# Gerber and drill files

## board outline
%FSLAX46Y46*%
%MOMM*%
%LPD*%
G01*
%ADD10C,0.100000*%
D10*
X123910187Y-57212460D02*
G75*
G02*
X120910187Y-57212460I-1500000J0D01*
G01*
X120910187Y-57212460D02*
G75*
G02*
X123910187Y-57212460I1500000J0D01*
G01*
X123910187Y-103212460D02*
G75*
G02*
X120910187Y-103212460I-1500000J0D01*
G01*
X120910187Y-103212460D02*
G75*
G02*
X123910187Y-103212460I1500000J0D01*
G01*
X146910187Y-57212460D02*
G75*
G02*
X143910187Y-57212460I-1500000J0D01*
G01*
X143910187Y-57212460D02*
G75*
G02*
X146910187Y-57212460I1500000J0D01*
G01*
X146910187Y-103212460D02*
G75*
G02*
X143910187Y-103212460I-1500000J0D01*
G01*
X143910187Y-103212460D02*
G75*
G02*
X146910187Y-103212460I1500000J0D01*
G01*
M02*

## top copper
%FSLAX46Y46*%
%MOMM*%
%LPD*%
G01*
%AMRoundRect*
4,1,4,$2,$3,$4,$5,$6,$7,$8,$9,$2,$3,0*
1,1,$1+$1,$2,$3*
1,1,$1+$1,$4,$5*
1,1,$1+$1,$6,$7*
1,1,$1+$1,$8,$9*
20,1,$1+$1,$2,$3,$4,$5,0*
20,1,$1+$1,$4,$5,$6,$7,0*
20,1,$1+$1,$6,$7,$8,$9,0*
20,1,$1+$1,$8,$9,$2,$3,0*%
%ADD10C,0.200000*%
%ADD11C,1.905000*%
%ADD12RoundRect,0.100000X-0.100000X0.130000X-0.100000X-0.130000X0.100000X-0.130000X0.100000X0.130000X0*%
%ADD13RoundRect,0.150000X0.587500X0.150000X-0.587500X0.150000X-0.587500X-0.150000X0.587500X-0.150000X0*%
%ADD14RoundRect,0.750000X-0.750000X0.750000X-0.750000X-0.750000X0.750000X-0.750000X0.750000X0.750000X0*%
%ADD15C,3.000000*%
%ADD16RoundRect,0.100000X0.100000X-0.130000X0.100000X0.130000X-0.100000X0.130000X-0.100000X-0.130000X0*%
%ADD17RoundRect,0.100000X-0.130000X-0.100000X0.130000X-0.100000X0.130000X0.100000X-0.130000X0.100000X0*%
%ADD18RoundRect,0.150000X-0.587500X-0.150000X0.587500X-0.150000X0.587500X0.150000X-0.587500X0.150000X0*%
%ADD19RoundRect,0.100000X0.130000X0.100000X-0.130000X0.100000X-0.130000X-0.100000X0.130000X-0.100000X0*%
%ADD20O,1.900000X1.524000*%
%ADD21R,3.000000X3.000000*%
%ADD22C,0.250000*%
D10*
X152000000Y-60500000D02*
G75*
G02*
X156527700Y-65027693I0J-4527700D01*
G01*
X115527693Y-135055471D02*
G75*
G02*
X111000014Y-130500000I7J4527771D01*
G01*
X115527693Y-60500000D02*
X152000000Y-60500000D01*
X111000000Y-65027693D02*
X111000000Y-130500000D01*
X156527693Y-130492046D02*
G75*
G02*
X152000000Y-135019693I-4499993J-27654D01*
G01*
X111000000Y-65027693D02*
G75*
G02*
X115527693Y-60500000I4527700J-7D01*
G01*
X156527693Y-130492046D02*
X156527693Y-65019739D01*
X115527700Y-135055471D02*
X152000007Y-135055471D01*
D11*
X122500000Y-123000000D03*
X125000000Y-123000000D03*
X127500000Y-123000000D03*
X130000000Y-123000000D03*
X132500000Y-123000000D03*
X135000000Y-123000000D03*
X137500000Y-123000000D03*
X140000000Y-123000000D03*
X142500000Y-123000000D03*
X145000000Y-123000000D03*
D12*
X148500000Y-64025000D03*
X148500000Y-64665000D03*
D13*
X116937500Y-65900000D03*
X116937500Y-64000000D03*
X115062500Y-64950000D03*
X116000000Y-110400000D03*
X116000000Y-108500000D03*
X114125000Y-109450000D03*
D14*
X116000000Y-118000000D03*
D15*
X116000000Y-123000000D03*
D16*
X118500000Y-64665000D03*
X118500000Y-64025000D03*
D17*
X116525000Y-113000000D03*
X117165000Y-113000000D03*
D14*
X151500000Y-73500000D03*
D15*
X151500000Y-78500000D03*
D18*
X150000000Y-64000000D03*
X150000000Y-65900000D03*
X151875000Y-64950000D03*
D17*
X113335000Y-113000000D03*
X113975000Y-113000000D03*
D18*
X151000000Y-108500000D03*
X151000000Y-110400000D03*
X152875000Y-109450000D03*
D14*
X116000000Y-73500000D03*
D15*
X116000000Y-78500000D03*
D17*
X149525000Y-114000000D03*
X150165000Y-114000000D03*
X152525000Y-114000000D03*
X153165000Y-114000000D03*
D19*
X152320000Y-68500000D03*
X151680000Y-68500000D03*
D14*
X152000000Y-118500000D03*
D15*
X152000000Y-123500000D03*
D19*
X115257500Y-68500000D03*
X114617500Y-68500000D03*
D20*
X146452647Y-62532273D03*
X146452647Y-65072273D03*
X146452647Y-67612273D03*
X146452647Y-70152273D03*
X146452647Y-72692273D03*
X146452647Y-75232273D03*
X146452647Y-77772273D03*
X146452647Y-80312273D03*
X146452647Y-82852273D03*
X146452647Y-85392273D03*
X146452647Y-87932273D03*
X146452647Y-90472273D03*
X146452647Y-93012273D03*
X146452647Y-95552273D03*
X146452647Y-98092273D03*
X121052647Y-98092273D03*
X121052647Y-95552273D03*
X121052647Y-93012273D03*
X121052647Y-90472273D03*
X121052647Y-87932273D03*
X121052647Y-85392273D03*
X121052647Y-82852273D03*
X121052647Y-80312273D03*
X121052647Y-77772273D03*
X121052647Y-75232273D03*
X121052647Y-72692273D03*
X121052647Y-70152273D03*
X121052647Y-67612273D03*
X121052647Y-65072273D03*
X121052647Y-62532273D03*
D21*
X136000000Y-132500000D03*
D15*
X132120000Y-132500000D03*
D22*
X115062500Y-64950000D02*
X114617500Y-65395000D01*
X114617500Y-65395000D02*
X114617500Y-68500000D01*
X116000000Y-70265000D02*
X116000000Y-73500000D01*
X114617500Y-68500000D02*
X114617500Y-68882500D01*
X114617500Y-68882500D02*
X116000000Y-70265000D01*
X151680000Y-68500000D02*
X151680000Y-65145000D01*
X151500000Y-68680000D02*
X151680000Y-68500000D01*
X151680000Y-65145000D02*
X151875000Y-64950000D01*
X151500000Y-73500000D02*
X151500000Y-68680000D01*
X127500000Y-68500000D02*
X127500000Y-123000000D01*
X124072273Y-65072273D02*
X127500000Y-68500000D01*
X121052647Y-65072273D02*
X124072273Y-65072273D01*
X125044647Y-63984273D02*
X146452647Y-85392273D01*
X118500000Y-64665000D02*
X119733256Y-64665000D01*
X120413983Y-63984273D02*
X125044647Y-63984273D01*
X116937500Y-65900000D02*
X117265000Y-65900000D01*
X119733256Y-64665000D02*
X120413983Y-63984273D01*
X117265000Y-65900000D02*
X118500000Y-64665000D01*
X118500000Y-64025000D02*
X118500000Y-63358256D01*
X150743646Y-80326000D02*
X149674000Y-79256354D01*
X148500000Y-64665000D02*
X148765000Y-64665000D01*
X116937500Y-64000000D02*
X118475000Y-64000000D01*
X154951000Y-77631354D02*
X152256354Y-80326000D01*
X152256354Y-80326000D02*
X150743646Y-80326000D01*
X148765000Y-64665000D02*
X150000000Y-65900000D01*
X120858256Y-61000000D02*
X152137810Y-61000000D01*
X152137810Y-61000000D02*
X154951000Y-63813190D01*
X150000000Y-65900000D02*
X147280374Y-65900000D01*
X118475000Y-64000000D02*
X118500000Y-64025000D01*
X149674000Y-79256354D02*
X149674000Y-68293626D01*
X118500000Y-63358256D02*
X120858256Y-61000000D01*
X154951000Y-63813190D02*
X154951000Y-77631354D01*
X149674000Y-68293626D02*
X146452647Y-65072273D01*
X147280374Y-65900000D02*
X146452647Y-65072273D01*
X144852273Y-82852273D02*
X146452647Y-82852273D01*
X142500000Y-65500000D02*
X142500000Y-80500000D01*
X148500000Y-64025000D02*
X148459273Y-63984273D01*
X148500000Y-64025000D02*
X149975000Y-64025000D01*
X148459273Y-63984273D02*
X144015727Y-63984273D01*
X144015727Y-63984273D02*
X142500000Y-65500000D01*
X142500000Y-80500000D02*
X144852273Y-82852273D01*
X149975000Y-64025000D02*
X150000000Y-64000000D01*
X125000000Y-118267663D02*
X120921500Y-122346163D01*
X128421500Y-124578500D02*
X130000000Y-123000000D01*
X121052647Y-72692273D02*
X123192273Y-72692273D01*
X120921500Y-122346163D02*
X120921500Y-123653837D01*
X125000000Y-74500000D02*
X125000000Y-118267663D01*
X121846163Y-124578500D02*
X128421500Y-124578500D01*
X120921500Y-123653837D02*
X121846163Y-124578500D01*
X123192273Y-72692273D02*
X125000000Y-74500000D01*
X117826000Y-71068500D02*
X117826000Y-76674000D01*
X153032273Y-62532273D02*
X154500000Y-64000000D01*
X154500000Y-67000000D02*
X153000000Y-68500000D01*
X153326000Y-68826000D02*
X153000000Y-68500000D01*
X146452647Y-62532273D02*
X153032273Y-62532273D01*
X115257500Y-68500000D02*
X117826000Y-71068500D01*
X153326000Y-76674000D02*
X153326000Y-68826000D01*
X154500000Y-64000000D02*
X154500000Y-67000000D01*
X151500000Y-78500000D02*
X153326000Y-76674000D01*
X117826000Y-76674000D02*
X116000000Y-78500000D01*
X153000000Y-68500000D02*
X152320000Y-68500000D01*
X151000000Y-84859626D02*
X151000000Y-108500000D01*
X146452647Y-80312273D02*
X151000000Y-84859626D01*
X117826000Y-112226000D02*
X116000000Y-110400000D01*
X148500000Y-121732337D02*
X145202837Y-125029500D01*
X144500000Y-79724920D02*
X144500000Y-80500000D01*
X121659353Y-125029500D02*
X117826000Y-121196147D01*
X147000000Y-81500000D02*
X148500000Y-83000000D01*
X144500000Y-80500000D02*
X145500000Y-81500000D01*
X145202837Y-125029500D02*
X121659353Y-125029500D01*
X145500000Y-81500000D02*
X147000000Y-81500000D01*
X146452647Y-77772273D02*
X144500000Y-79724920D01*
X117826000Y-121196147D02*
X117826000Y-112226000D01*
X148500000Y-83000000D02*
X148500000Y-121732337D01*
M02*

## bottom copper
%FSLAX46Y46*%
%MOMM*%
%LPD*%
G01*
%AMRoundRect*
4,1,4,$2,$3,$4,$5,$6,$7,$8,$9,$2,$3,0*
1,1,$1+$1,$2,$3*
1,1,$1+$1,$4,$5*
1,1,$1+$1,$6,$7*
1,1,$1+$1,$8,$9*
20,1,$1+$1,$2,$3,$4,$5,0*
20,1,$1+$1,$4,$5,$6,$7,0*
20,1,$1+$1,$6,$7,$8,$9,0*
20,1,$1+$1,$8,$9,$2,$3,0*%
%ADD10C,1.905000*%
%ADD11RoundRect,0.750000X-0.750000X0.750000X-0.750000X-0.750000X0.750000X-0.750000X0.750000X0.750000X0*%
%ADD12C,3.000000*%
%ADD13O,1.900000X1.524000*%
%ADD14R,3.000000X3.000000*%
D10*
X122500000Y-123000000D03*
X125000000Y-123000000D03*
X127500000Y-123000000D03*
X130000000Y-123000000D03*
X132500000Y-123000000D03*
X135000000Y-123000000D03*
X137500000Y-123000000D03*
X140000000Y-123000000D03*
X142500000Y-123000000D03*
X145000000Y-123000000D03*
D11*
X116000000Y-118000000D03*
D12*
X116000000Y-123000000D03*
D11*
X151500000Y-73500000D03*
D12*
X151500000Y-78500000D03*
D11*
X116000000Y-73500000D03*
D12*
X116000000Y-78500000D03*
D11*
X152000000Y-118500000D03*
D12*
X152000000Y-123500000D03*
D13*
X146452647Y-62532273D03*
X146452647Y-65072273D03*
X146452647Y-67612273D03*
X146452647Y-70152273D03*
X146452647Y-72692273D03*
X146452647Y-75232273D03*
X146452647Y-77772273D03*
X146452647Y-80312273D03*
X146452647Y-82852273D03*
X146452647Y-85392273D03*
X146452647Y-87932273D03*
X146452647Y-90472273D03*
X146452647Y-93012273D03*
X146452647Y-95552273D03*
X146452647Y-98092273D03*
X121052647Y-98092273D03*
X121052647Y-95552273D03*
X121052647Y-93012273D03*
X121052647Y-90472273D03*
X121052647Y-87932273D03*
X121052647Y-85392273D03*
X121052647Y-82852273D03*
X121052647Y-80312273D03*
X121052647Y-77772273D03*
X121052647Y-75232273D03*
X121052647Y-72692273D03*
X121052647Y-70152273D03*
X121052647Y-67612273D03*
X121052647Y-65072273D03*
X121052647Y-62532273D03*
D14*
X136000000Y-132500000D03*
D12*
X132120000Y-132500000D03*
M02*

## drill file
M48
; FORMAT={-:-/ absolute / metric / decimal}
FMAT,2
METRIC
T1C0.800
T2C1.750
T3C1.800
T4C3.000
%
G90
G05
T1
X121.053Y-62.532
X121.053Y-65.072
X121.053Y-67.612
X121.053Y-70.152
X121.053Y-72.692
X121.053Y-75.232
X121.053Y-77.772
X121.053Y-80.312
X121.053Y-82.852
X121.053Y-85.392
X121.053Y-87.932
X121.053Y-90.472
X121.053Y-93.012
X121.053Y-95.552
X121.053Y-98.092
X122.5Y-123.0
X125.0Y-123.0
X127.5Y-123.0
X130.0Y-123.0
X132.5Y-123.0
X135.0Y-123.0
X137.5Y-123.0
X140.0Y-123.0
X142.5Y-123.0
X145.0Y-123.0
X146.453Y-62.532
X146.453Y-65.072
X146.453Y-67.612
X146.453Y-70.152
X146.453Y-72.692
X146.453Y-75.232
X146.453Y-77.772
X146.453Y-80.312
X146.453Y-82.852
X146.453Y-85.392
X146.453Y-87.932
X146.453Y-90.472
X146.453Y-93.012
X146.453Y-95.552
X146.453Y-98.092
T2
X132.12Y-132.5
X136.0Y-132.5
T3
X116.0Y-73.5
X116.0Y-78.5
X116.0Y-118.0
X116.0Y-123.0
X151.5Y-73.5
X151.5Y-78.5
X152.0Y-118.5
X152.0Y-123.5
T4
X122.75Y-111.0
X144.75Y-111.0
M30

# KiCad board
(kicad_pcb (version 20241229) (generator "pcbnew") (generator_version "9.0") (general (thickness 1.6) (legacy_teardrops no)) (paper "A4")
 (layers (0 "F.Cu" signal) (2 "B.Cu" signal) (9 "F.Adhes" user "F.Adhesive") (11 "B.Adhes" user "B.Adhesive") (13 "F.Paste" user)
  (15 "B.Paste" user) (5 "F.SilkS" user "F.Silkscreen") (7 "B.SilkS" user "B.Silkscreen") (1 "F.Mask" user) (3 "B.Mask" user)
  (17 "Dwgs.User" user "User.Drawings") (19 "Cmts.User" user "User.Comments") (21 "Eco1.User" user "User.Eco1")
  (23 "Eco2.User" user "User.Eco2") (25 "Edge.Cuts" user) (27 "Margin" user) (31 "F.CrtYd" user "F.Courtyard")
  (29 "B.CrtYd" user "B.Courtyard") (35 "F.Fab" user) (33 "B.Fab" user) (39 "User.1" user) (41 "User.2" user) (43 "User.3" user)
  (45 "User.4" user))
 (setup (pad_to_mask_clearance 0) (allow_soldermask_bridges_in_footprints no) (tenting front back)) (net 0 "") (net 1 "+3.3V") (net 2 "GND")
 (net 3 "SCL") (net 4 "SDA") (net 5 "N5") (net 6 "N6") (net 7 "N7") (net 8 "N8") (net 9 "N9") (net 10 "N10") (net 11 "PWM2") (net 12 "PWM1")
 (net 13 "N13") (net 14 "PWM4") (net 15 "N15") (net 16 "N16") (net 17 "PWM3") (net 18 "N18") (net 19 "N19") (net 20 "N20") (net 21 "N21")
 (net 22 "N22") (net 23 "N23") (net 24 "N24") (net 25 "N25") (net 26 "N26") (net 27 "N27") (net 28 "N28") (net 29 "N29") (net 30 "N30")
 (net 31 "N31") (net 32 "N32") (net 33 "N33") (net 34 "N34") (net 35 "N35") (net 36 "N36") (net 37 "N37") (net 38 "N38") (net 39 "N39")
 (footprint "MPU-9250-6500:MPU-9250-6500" (layer "F.Cu") (at 120.75 125 90)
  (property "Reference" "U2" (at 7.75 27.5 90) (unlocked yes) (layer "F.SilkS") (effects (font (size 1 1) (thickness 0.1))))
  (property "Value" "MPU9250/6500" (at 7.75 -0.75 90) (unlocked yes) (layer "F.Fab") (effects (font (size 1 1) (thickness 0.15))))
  (pad "" np_thru_hole circle (at 14 2 90) (size 3 3) (drill 3) (layers "*.Cu" "*.Mask") (clearance 0.5))
  (pad "" np_thru_hole circle (at 14 24 90) (size 3 3) (drill 3) (layers "*.Cu" "*.Mask") (clearance 0.5))
  (pad "1" thru_hole circle (at 2 1.75 90) (size 1.905 1.905) (drill 0.8) (layers "*.Cu" "*.Mask") (remove_unused_layers no) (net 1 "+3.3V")
   (clearance 0.5))
  (pad "2" thru_hole circle (at 2 4.25 90) (size 1.905 1.905) (drill 0.8) (layers "*.Cu" "*.Mask") (remove_unused_layers no) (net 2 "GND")
   (clearance 0.5))
  (pad "3" thru_hole circle (at 2 6.75 90) (size 1.905 1.905) (drill 0.8) (layers "*.Cu" "*.Mask") (remove_unused_layers no) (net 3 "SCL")
   (clearance 0.5))
  (pad "4" thru_hole circle (at 2 9.25 90) (size 1.905 1.905) (drill 0.8) (layers "*.Cu" "*.Mask") (remove_unused_layers no) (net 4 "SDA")
   (clearance 0.5))
  (pad "5" thru_hole circle (at 2 11.75 90) (size 1.905 1.905) (drill 0.8) (layers "*.Cu" "*.Mask") (remove_unused_layers no) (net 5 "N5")
   (clearance 0.5))
  (pad "6" thru_hole circle (at 2 14.25 90) (size 1.905 1.905) (drill 0.8) (layers "*.Cu" "*.Mask") (remove_unused_layers no) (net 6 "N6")
   (clearance 0.5))
  (pad "7" thru_hole circle (at 2 16.75 90) (size 1.905 1.905) (drill 0.8) (layers "*.Cu" "*.Mask") (remove_unused_layers no) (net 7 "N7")
   (clearance 0.5))
  (pad "8" thru_hole circle (at 2 19.25 90) (size 1.905 1.905) (drill 0.8) (layers "*.Cu" "*.Mask") (remove_unused_layers no) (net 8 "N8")
   (clearance 0.5))
  (pad "9" thru_hole circle (at 2 21.75 90) (size 1.905 1.905) (drill 0.8) (layers "*.Cu" "*.Mask") (remove_unused_layers no) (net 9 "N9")
   (clearance 0.5))
  (pad "10" thru_hole circle (at 2 24.25 90) (size 1.905 1.905) (drill 0.8) (layers "*.Cu" "*.Mask") (remove_unused_layers no)
   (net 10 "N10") (clearance 0.5)))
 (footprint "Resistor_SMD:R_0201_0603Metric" (layer "F.Cu") (at 148.5 64.345 -90)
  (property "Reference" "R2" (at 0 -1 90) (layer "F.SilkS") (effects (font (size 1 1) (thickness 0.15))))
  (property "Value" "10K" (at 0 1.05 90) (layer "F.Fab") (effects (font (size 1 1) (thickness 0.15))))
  (pad "" smd roundrect (at -0.345 0 270) (size 0.318 0.36) (layers "F.Paste") (roundrect_rratio 0.25))
  (pad "" smd roundrect (at 0.345 0 270) (size 0.318 0.36) (layers "F.Paste") (roundrect_rratio 0.25))
  (pad "1" smd roundrect (at -0.32 0 270) (size 0.46 0.4) (layers "F.Cu" "F.Mask") (roundrect_rratio 0.25) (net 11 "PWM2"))
  (pad "2" smd roundrect (at 0.32 0 270) (size 0.46 0.4) (layers "F.Cu" "F.Mask") (roundrect_rratio 0.25) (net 2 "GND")))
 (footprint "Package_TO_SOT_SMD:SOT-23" (layer "F.Cu") (at 116 64.95 180)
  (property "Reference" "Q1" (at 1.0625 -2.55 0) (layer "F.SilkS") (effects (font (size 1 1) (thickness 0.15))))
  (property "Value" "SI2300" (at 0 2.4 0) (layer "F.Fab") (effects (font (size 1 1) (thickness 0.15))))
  (pad "1" smd roundrect (at -0.9375 -0.95 180) (size 1.475 0.6) (layers "F.Cu" "F.Mask" "F.Paste") (roundrect_rratio 0.25) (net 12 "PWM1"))
  (pad "2" smd roundrect (at -0.9375 0.95 180) (size 1.475 0.6) (layers "F.Cu" "F.Mask" "F.Paste") (roundrect_rratio 0.25) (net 2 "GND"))
  (pad "3" smd roundrect (at 0.9375 0 180) (size 1.475 0.6) (layers "F.Cu" "F.Mask" "F.Paste") (roundrect_rratio 0.25) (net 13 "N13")))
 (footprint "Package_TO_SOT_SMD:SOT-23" (layer "F.Cu") (at 115.0625 109.45 180)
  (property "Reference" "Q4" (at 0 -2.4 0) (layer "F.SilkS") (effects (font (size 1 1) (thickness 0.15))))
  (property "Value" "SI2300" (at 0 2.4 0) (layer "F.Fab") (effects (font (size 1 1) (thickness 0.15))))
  (pad "1" smd roundrect (at -0.9375 -0.95 180) (size 1.475 0.6) (layers "F.Cu" "F.Mask" "F.Paste") (roundrect_rratio 0.25) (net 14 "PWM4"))
  (pad "2" smd roundrect (at -0.9375 0.95 180) (size 1.475 0.6) (layers "F.Cu" "F.Mask" "F.Paste") (roundrect_rratio 0.25) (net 2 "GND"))
  (pad "3" smd roundrect (at 0.9375 0 180) (size 1.475 0.6) (layers "F.Cu" "F.Mask" "F.Paste") (roundrect_rratio 0.25) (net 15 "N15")))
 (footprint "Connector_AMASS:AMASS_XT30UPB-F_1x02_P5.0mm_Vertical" (layer "F.Cu") (at 116 118 -90)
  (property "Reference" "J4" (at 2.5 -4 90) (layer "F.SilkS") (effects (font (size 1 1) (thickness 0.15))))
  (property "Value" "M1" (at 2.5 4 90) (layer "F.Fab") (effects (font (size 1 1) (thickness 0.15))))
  (pad "1" thru_hole roundrect (at 0 0 270) (size 3 3) (drill 1.8) (layers "*.Cu" "*.Mask") (remove_unused_layers no)
   (roundrect_rratio 0.25) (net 15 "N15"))
  (pad "2" thru_hole circle (at 5 0 270) (size 3 3) (drill 1.8) (layers "*.Cu" "*.Mask") (remove_unused_layers no) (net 1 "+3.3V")))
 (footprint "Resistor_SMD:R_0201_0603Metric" (layer "F.Cu") (at 118.5 64.345 90)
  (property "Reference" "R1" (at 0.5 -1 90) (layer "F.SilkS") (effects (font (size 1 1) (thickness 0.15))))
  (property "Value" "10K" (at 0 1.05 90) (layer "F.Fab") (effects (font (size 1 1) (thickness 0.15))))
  (pad "" smd roundrect (at -0.345 0 90) (size 0.318 0.36) (layers "F.Paste") (roundrect_rratio 0.25))
  (pad "" smd roundrect (at 0.345 0 90) (size 0.318 0.36) (layers "F.Paste") (roundrect_rratio 0.25))
  (pad "1" smd roundrect (at -0.32 0 90) (size 0.46 0.4) (layers "F.Cu" "F.Mask") (roundrect_rratio 0.25) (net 12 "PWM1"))
  (pad "2" smd roundrect (at 0.32 0 90) (size 0.46 0.4) (layers "F.Cu" "F.Mask") (roundrect_rratio 0.25) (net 2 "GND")))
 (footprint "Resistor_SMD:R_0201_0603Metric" (layer "F.Cu") (at 116.845 113)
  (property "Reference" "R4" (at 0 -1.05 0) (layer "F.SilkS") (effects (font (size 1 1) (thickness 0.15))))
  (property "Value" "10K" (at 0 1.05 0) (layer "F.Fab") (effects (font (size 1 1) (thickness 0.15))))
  (pad "" smd roundrect (at -0.345 0) (size 0.318 0.36) (layers "F.Paste") (roundrect_rratio 0.25))
  (pad "" smd roundrect (at 0.345 0) (size 0.318 0.36) (layers "F.Paste") (roundrect_rratio 0.25))
  (pad "1" smd roundrect (at -0.32 0) (size 0.46 0.4) (layers "F.Cu" "F.Mask") (roundrect_rratio 0.25) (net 14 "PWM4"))
  (pad "2" smd roundrect (at 0.32 0) (size 0.46 0.4) (layers "F.Cu" "F.Mask") (roundrect_rratio 0.25) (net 2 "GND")))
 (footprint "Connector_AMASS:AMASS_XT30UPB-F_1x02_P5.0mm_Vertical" (layer "F.Cu") (at 151.5 73.5 -90)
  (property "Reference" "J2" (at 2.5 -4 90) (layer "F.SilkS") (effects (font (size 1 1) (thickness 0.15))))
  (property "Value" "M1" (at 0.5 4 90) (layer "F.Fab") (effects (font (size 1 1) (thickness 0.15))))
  (pad "1" thru_hole roundrect (at 0 0 270) (size 3 3) (drill 1.8) (layers "*.Cu" "*.Mask") (remove_unused_layers no)
   (roundrect_rratio 0.25) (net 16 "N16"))
  (pad "2" thru_hole circle (at 5 0 270) (size 3 3) (drill 1.8) (layers "*.Cu" "*.Mask") (remove_unused_layers no) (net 1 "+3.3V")))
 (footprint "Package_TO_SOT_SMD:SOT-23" (layer "F.Cu") (at 150.9375 64.95)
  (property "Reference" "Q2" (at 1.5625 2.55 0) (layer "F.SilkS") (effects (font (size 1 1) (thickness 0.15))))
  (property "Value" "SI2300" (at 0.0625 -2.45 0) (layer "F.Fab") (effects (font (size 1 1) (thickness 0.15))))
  (pad "1" smd roundrect (at -0.9375 -0.95) (size 1.475 0.6) (layers "F.Cu" "F.Mask" "F.Paste") (roundrect_rratio 0.25) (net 11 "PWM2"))
  (pad "2" smd roundrect (at -0.9375 0.95) (size 1.475 0.6) (layers "F.Cu" "F.Mask" "F.Paste") (roundrect_rratio 0.25) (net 2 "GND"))
  (pad "3" smd roundrect (at 0.9375 0) (size 1.475 0.6) (layers "F.Cu" "F.Mask" "F.Paste") (roundrect_rratio 0.25) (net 16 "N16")))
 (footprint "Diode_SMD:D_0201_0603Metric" (layer "F.Cu") (at 113.655 113)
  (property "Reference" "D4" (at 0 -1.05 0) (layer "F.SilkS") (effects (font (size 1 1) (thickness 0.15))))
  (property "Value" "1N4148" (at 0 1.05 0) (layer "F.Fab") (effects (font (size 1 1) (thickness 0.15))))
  (pad "" smd roundrect (at -0.345 0) (size 0.318 0.36) (layers "F.Paste") (roundrect_rratio 0.25))
  (pad "" smd roundrect (at 0.345 0) (size 0.318 0.36) (layers "F.Paste") (roundrect_rratio 0.25))
  (pad "1" smd roundrect (at -0.32 0) (size 0.46 0.4) (layers "F.Cu" "F.Mask") (roundrect_rratio 0.25) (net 1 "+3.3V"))
  (pad "2" smd roundrect (at 0.32 0) (size 0.46 0.4) (layers "F.Cu" "F.Mask") (roundrect_rratio 0.25) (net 15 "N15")))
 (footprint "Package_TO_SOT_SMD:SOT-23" (layer "F.Cu") (at 151.9375 109.45)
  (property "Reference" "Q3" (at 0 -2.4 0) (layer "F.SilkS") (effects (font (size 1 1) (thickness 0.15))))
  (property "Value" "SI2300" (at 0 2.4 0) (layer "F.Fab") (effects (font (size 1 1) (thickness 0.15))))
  (pad "1" smd roundrect (at -0.9375 -0.95) (size 1.475 0.6) (layers "F.Cu" "F.Mask" "F.Paste") (roundrect_rratio 0.25) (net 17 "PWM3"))
  (pad "2" smd roundrect (at -0.9375 0.95) (size 1.475 0.6) (layers "F.Cu" "F.Mask" "F.Paste") (roundrect_rratio 0.25) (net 2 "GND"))
  (pad "3" smd roundrect (at 0.9375 0) (size 1.475 0.6) (layers "F.Cu" "F.Mask" "F.Paste") (roundrect_rratio 0.25) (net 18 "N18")))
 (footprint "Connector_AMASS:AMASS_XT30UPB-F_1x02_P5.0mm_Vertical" (layer "F.Cu") (at 116 73.5 -90)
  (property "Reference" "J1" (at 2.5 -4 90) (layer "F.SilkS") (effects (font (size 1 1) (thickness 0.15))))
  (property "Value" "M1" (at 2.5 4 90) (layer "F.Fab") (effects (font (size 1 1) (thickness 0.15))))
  (pad "1" thru_hole roundrect (at 0 0 270) (size 3 3) (drill 1.8) (layers "*.Cu" "*.Mask") (remove_unused_layers no)
   (roundrect_rratio 0.25) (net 13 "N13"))
  (pad "2" thru_hole circle (at 5 0 270) (size 3 3) (drill 1.8) (layers "*.Cu" "*.Mask") (remove_unused_layers no) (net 1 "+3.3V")))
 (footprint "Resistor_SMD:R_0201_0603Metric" (layer "F.Cu") (at 149.845 114)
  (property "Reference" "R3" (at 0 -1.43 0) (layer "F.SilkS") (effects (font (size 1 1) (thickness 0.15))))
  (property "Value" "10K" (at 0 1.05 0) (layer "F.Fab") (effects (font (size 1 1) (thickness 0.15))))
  (pad "" smd roundrect (at -0.345 0) (size 0.318 0.36) (layers "F.Paste") (roundrect_rratio 0.25))
  (pad "" smd roundrect (at 0.345 0) (size 0.318 0.36) (layers "F.Paste") (roundrect_rratio 0.25))
  (pad "1" smd roundrect (at -0.32 0) (size 0.46 0.4) (layers "F.Cu" "F.Mask") (roundrect_rratio 0.25) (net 17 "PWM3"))
  (pad "2" smd roundrect (at 0.32 0) (size 0.46 0.4) (layers "F.Cu" "F.Mask") (roundrect_rratio 0.25) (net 2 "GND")))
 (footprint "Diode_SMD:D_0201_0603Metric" (layer "F.Cu") (at 152.845 114)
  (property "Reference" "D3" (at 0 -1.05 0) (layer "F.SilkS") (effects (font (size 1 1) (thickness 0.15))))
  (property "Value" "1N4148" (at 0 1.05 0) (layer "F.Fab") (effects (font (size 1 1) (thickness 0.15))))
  (pad "" smd roundrect (at -0.345 0) (size 0.318 0.36) (layers "F.Paste") (roundrect_rratio 0.25))
  (pad "" smd roundrect (at 0.345 0) (size 0.318 0.36) (layers "F.Paste") (roundrect_rratio 0.25))
  (pad "1" smd roundrect (at -0.32 0) (size 0.46 0.4) (layers "F.Cu" "F.Mask") (roundrect_rratio 0.25) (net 1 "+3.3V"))
  (pad "2" smd roundrect (at 0.32 0) (size 0.46 0.4) (layers "F.Cu" "F.Mask") (roundrect_rratio 0.25) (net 18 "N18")))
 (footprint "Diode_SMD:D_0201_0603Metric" (layer "F.Cu") (at 152 68.5 180)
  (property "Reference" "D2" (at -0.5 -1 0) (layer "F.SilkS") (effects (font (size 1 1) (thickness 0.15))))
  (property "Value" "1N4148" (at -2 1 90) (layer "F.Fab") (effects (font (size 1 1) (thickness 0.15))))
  (pad "" smd roundrect (at -0.345 0 180) (size 0.318 0.36) (layers "F.Paste") (roundrect_rratio 0.25))
  (pad "" smd roundrect (at 0.345 0 180) (size 0.318 0.36) (layers "F.Paste") (roundrect_rratio 0.25))
  (pad "1" smd roundrect (at -0.32 0 180) (size 0.46 0.4) (layers "F.Cu" "F.Mask") (roundrect_rratio 0.25) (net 1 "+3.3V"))
  (pad "2" smd roundrect (at 0.32 0 180) (size 0.46 0.4) (layers "F.Cu" "F.Mask") (roundrect_rratio 0.25) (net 16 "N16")))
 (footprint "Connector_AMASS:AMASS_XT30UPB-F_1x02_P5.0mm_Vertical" (layer "F.Cu") (at 152 118.5 -90)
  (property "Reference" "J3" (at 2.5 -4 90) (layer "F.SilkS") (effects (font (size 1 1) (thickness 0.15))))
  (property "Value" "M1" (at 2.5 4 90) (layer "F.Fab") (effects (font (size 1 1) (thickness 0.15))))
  (pad "1" thru_hole roundrect (at 0 0 270) (size 3 3) (drill 1.8) (layers "*.Cu" "*.Mask") (remove_unused_layers no)
   (roundrect_rratio 0.25) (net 18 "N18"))
  (pad "2" thru_hole circle (at 5 0 270) (size 3 3) (drill 1.8) (layers "*.Cu" "*.Mask") (remove_unused_layers no) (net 1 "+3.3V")))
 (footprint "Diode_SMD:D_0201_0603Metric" (layer "F.Cu") (at 114.9375 68.5 180)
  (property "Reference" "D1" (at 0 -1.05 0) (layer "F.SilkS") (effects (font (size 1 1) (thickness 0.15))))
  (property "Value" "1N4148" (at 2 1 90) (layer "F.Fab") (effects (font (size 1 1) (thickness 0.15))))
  (pad "" smd roundrect (at -0.345 0 180) (size 0.318 0.36) (layers "F.Paste") (roundrect_rratio 0.25))
  (pad "" smd roundrect (at 0.345 0 180) (size 0.318 0.36) (layers "F.Paste") (roundrect_rratio 0.25))
  (pad "1" smd roundrect (at -0.32 0 180) (size 0.46 0.4) (layers "F.Cu" "F.Mask") (roundrect_rratio 0.25) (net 1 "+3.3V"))
  (pad "2" smd roundrect (at 0.32 0 180) (size 0.46 0.4) (layers "F.Cu" "F.Mask") (roundrect_rratio 0.25) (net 13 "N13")))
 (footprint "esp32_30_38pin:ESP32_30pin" (layer "F.Cu") (at 133.980187 80.07246 -90)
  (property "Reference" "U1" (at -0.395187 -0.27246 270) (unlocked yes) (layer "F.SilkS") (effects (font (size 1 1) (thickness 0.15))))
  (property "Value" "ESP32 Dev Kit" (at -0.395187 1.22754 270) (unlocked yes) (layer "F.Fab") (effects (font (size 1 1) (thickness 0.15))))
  (fp_circle (center -22.86 11.57) (end -21.36 11.57) (stroke (width 0.1) (type default)) (fill no) (layer "Edge.Cuts"))
  (fp_circle (center 23.14 11.57) (end 24.64 11.57) (stroke (width 0.1) (type default)) (fill no) (layer "Edge.Cuts"))
  (fp_circle (center -22.86 -11.43) (end -21.36 -11.43) (stroke (width 0.1) (type default)) (fill no) (layer "Edge.Cuts"))
  (fp_circle (center 23.14 -11.43) (end 24.64 -11.43) (stroke (width 0.1) (type default)) (fill no) (layer "Edge.Cuts"))
  (pad "1" thru_hole oval (at -17.540187 -12.47246 270) (size 1.524 1.9) (drill 0.8) (layers "*.Cu" "*.Mask") (remove_unused_layers no)
   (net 1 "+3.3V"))
  (pad "2" thru_hole oval (at -15.000187 -12.47246 270) (size 1.524 1.9) (drill 0.8) (layers "*.Cu" "*.Mask") (remove_unused_layers no)
   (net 2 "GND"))
  (pad "3" thru_hole oval (at -12.460187 -12.47246 270) (size 1.524 1.9) (drill 0.8) (layers "*.Cu" "*.Mask") (remove_unused_layers no)
   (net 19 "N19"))
  (pad "4" thru_hole oval (at -9.920187 -12.47246 270) (size 1.524 1.9) (drill 0.8) (layers "*.Cu" "*.Mask") (remove_unused_layers no)
   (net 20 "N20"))
  (pad "5" thru_hole oval (at -7.380187 -12.47246 270) (size 1.524 1.9) (drill 0.8) (layers "*.Cu" "*.Mask") (remove_unused_layers no)
   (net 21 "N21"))
  (pad "6" thru_hole oval (at -4.840187 -12.47246 270) (size 1.524 1.9) (drill 0.8) (layers "*.Cu" "*.Mask") (remove_unused_layers no)
   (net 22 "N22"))
  (pad "7" thru_hole oval (at -2.300187 -12.47246 270) (size 1.524 1.9) (drill 0.8) (layers "*.Cu" "*.Mask") (remove_unused_layers no)
   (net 14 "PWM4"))
  (pad "8" thru_hole oval (at 0.239813 -12.47246 270) (size 1.524 1.9) (drill 0.8) (layers "*.Cu" "*.Mask") (remove_unused_layers no)
   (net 17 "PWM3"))
  (pad "9" thru_hole oval (at 2.779813 -12.47246 270) (size 1.524 1.9) (drill 0.8) (layers "*.Cu" "*.Mask") (remove_unused_layers no)
   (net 11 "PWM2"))
  (pad "10" thru_hole oval (at 5.319813 -12.47246 270) (size 1.524 1.9) (drill 0.8) (layers "*.Cu" "*.Mask") (remove_unused_layers no)
   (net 12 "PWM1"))
  (pad "11" thru_hole oval (at 7.859813 -12.47246 270) (size 1.524 1.9) (drill 0.8) (layers "*.Cu" "*.Mask") (remove_unused_layers no)
   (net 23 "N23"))
  (pad "12" thru_hole oval (at 10.399813 -12.47246 270) (size 1.524 1.9) (drill 0.8) (layers "*.Cu" "*.Mask") (remove_unused_layers no)
   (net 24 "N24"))
  (pad "13" thru_hole oval (at 12.939813 -12.47246 270) (size 1.524 1.9) (drill 0.8) (layers "*.Cu" "*.Mask") (remove_unused_layers no)
   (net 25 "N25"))
  (pad "14" thru_hole oval (at 15.479813 -12.47246 270) (size 1.524 1.9) (drill 0.8) (layers "*.Cu" "*.Mask") (remove_unused_layers no)
   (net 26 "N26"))
  (pad "15" thru_hole oval (at 18.019813 -12.47246 270) (size 1.524 1.9) (drill 0.8) (layers "*.Cu" "*.Mask") (remove_unused_layers no)
   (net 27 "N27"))
  (pad "16" thru_hole oval (at 18.019813 12.92754 270) (size 1.524 1.9) (drill 0.8) (layers "*.Cu" "*.Mask") (remove_unused_layers no)
   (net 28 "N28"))
  (pad "17" thru_hole oval (at 15.479813 12.92754 270) (size 1.524 1.9) (drill 0.8) (layers "*.Cu" "*.Mask") (remove_unused_layers no)
   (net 2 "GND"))
  (pad "18" thru_hole oval (at 12.939813 12.92754 270) (size 1.524 1.9) (drill 0.8) (layers "*.Cu" "*.Mask") (remove_unused_layers no)
   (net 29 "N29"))
  (pad "19" thru_hole oval (at 10.399813 12.92754 270) (size 1.524 1.9) (drill 0.8) (layers "*.Cu" "*.Mask") (remove_unused_layers no)
   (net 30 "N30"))
  (pad "20" thru_hole oval (at 7.859813 12.92754 270) (size 1.524 1.9) (drill 0.8) (layers "*.Cu" "*.Mask") (remove_unused_layers no)
   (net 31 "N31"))
  (pad "21" thru_hole oval (at 5.319813 12.92754 270) (size 1.524 1.9) (drill 0.8) (layers "*.Cu" "*.Mask") (remove_unused_layers no)
   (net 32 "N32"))
  (pad "22" thru_hole oval (at 2.779813 12.92754 270) (size 1.524 1.9) (drill 0.8) (layers "*.Cu" "*.Mask") (remove_unused_layers no)
   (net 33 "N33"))
  (pad "23" thru_hole oval (at 0.239813 12.92754 270) (size 1.524 1.9) (drill 0.8) (layers "*.Cu" "*.Mask") (remove_unused_layers no)
   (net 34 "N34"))
  (pad "24" thru_hole oval (at -2.300187 12.92754 270) (size 1.524 1.9) (drill 0.8) (layers "*.Cu" "*.Mask") (remove_unused_layers no)
   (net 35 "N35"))
  (pad "25" thru_hole oval (at -4.840187 12.92754 270) (size 1.524 1.9) (drill 0.8) (layers "*.Cu" "*.Mask") (remove_unused_layers no)
   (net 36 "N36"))
  (pad "26" thru_hole oval (at -7.380187 12.92754 270) (size 1.524 1.9) (drill 0.8) (layers "*.Cu" "*.Mask") (remove_unused_layers no)
   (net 4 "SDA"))
  (pad "27" thru_hole oval (at -9.920187 12.92754 270) (size 1.524 1.9) (drill 0.8) (layers "*.Cu" "*.Mask") (remove_unused_layers no)
   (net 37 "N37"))
  (pad "28" thru_hole oval (at -12.460187 12.92754 270) (size 1.524 1.9) (drill 0.8) (layers "*.Cu" "*.Mask") (remove_unused_layers no)
   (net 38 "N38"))
  (pad "29" thru_hole oval (at -15.000187 12.92754 270) (size 1.524 1.9) (drill 0.8) (layers "*.Cu" "*.Mask") (remove_unused_layers no)
   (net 3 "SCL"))
  (pad "30" thru_hole oval (at -17.540187 12.92754 270) (size 1.524 1.9) (drill 0.8) (layers "*.Cu" "*.Mask") (remove_unused_layers no)
   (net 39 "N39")))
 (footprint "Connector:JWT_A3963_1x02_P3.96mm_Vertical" (layer "F.Cu") (at 136 132.5 180)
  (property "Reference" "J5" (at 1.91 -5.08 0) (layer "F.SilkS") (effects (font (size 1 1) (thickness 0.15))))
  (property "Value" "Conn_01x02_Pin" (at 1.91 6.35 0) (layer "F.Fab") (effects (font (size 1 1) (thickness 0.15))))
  (pad "1" thru_hole rect (at 0 0 180) (size 3 3) (drill 1.75) (layers "*.Cu" "*.Mask") (remove_unused_layers no) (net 1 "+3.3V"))
  (pad "2" thru_hole circle (at 3.88 0 180) (size 3 3) (drill 1.75) (layers "*.Cu" "*.Mask") (remove_unused_layers no) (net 2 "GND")))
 (gr_arc (start 152 60.5) (mid 155.201562 61.826131) (end 156.527693 65.027693) (stroke (width 0.2) (type default)) (layer "F.Cu"))
 (gr_arc (start 115.527693 135.055471) (mid 112.316294 133.71951) (end 111 130.5) (stroke (width 0.2) (type default)) (layer "F.Cu"))
 (gr_line (start 115.527693 60.5) (end 152 60.5) (stroke (width 0.2) (type default)) (layer "F.Cu"))
 (gr_line (start 111 65.027693) (end 111 130.5) (stroke (width 0.2) (type default)) (layer "F.Cu"))
 (gr_arc (start 156.527693 130.492046) (mid 155.209734 133.70178) (end 152 135.019739) (stroke (width 0.2) (type default)) (layer "F.Cu"))
 (gr_arc (start 111 65.027693) (mid 112.326131 61.826131) (end 115.527693 60.5) (stroke (width 0.2) (type default)) (layer "F.Cu"))
 (gr_line (start 156.527693 130.492046) (end 156.527693 65.019739) (stroke (width 0.2) (type default)) (layer "F.Cu"))
 (gr_line (start 115.5277 135.055471) (end 152.000007 135.055471) (stroke (width 0.2) (type solid)) (layer "F.Cu"))
 (segment (start 115.0625 64.95) (end 114.6175 65.395) (width 0.25) (layer "F.Cu") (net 13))
 (segment (start 114.6175 65.395) (end 114.6175 68.5) (width 0.25) (layer "F.Cu") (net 13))
 (segment (start 116 70.265) (end 116 73.5) (width 0.25) (layer "F.Cu") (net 13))
 (segment (start 114.6175 68.5) (end 114.6175 68.8825) (width 0.25) (layer "F.Cu") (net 13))
 (segment (start 114.6175 68.8825) (end 116 70.265) (width 0.25) (layer "F.Cu") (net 13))
 (segment (start 151.68 68.5) (end 151.68 65.145) (width 0.25) (layer "F.Cu") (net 16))
 (segment (start 151.5 68.68) (end 151.68 68.5) (width 0.25) (layer "F.Cu") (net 16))
 (segment (start 151.68 65.145) (end 151.875 64.95) (width 0.25) (layer "F.Cu") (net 16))
 (segment (start 151.5 73.5) (end 151.5 68.68) (width 0.25) (layer "F.Cu") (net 16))
 (segment (start 127.5 68.5) (end 127.5 123) (width 0.25) (layer "F.Cu") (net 3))
 (segment (start 124.072273 65.072273) (end 127.5 68.5) (width 0.25) (layer "F.Cu") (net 3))
 (segment (start 121.052647 65.072273) (end 124.072273 65.072273) (width 0.25) (layer "F.Cu") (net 3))
 (segment (start 125.044647 63.984273) (end 146.452647 85.392273) (width 0.25) (layer "F.Cu") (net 12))
 (segment (start 118.5 64.665) (end 119.733256 64.665) (width 0.25) (layer "F.Cu") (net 12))
 (segment (start 120.413983 63.984273) (end 125.044647 63.984273) (width 0.25) (layer "F.Cu") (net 12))
 (segment (start 116.9375 65.9) (end 117.265 65.9) (width 0.25) (layer "F.Cu") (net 12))
 (segment (start 119.733256 64.665) (end 120.413983 63.984273) (width 0.25) (layer "F.Cu") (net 12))
 (segment (start 117.265 65.9) (end 118.5 64.665) (width 0.25) (layer "F.Cu") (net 12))
 (segment (start 118.5 64.025) (end 118.5 63.358256) (width 0.25) (layer "F.Cu") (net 2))
 (segment (start 150.743646 80.326) (end 149.674 79.256354) (width 0.25) (layer "F.Cu") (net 2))
 (segment (start 148.5 64.665) (end 148.765 64.665) (width 0.25) (layer "F.Cu") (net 2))
 (segment (start 116.9375 64) (end 118.475 64) (width 0.25) (layer "F.Cu") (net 2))
 (segment (start 154.951 77.631354) (end 152.256354 80.326) (width 0.25) (layer "F.Cu") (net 2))
 (segment (start 152.256354 80.326) (end 150.743646 80.326) (width 0.25) (layer "F.Cu") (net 2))
 (segment (start 148.765 64.665) (end 150 65.9) (width 0.25) (layer "F.Cu") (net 2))
 (segment (start 120.858256 61) (end 152.13781 61) (width 0.25) (layer "F.Cu") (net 2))
 (segment (start 152.13781 61) (end 154.951 63.81319) (width 0.25) (layer "F.Cu") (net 2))
 (segment (start 150 65.9) (end 147.280374 65.9) (width 0.25) (layer "F.Cu") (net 2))
 (segment (start 118.475 64) (end 118.5 64.025) (width 0.25) (layer "F.Cu") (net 2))
 (segment (start 149.674 79.256354) (end 149.674 68.293626) (width 0.25) (layer "F.Cu") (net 2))
 (segment (start 118.5 63.358256) (end 120.858256 61) (width 0.25) (layer "F.Cu") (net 2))
 (segment (start 154.951 63.81319) (end 154.951 77.631354) (width 0.25) (layer "F.Cu") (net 2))
 (segment (start 149.674 68.293626) (end 146.452647 65.072273) (width 0.25) (layer "F.Cu") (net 2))
 (segment (start 147.280374 65.9) (end 146.452647 65.072273) (width 0.25) (layer "F.Cu") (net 2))
 (segment (start 144.852273 82.852273) (end 146.452647 82.852273) (width 0.25) (layer "F.Cu") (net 11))
 (segment (start 142.5 65.5) (end 142.5 80.5) (width 0.25) (layer "F.Cu") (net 11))
 (segment (start 148.5 64.025) (end 148.459273 63.984273) (width 0.25) (layer "F.Cu") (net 11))
 (segment (start 148.5 64.025) (end 149.975 64.025) (width 0.25) (layer "F.Cu") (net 11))
 (segment (start 148.459273 63.984273) (end 144.015727 63.984273) (width 0.25) (layer "F.Cu") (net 11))
 (segment (start 144.015727 63.984273) (end 142.5 65.5) (width 0.25) (layer "F.Cu") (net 11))
 (segment (start 142.5 80.5) (end 144.852273 82.852273) (width 0.25) (layer "F.Cu") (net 11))
 (segment (start 149.975 64.025) (end 150 64) (width 0.25) (layer "F.Cu") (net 11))
 (segment (start 125 118.267663) (end 120.9215 122.346163) (width 0.25) (layer "F.Cu") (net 4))
 (segment (start 128.4215 124.5785) (end 130 123) (width 0.25) (layer "F.Cu") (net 4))
 (segment (start 121.052647 72.692273) (end 123.192273 72.692273) (width 0.25) (layer "F.Cu") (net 4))
 (segment (start 120.9215 122.346163) (end 120.9215 123.653837) (width 0.25) (layer "F.Cu") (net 4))
 (segment (start 125 74.5) (end 125 118.267663) (width 0.25) (layer "F.Cu") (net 4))
 (segment (start 121.846163 124.5785) (end 128.4215 124.5785) (width 0.25) (layer "F.Cu") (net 4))
 (segment (start 120.9215 123.653837) (end 121.846163 124.5785) (width 0.25) (layer "F.Cu") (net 4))
 (segment (start 123.192273 72.692273) (end 125 74.5) (width 0.25) (layer "F.Cu") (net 4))
 (segment (start 117.826 71.0685) (end 117.826 76.674) (width 0.25) (layer "F.Cu") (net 1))
 (segment (start 153.032273 62.532273) (end 154.5 64) (width 0.25) (layer "F.Cu") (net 1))
 (segment (start 154.5 67) (end 153 68.5) (width 0.25) (layer "F.Cu") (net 1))
 (segment (start 153.326 68.826) (end 153 68.5) (width 0.25) (layer "F.Cu") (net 1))
 (segment (start 146.452647 62.532273) (end 153.032273 62.532273) (width 0.25) (layer "F.Cu") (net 1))
 (segment (start 115.2575 68.5) (end 117.826 71.0685) (width 0.25) (layer "F.Cu") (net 1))
 (segment (start 153.326 76.674) (end 153.326 68.826) (width 0.25) (layer "F.Cu") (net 1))
 (segment (start 154.5 64) (end 154.5 67) (width 0.25) (layer "F.Cu") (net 1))
 (segment (start 151.5 78.5) (end 153.326 76.674) (width 0.25) (layer "F.Cu") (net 1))
 (segment (start 117.826 76.674) (end 116 78.5) (width 0.25) (layer "F.Cu") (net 1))
 (segment (start 153 68.5) (end 152.32 68.5) (width 0.25) (layer "F.Cu") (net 1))
 (segment (start 151 84.859626) (end 151 108.5) (width 0.25) (layer "F.Cu") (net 17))
 (segment (start 146.452647 80.312273) (end 151 84.859626) (width 0.25) (layer "F.Cu") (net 17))
 (segment (start 117.826 112.226) (end 116 110.4) (width 0.25) (layer "F.Cu") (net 14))
 (segment (start 148.5 121.732337) (end 145.202837 125.0295) (width 0.25) (layer "F.Cu") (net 14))
 (segment (start 144.5 79.72492) (end 144.5 80.5) (width 0.25) (layer "F.Cu") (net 14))
 (segment (start 121.659353 125.0295) (end 117.826 121.196147) (width 0.25) (layer "F.Cu") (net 14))
 (segment (start 147 81.5) (end 148.5 83) (width 0.25) (layer "F.Cu") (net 14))
 (segment (start 144.5 80.5) (end 145.5 81.5) (width 0.25) (layer "F.Cu") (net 14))
 (segment (start 145.202837 125.0295) (end 121.659353 125.0295) (width 0.25) (layer "F.Cu") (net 14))
 (segment (start 145.5 81.5) (end 147 81.5) (width 0.25) (layer "F.Cu") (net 14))
 (segment (start 146.452647 77.772273) (end 144.5 79.72492) (width 0.25) (layer "F.Cu") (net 14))
 (segment (start 117.826 121.196147) (end 117.826 112.226) (width 0.25) (layer "F.Cu") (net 14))
 (segment (start 148.5 83) (end 148.5 121.732337) (width 0.25) (layer "F.Cu") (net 14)))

